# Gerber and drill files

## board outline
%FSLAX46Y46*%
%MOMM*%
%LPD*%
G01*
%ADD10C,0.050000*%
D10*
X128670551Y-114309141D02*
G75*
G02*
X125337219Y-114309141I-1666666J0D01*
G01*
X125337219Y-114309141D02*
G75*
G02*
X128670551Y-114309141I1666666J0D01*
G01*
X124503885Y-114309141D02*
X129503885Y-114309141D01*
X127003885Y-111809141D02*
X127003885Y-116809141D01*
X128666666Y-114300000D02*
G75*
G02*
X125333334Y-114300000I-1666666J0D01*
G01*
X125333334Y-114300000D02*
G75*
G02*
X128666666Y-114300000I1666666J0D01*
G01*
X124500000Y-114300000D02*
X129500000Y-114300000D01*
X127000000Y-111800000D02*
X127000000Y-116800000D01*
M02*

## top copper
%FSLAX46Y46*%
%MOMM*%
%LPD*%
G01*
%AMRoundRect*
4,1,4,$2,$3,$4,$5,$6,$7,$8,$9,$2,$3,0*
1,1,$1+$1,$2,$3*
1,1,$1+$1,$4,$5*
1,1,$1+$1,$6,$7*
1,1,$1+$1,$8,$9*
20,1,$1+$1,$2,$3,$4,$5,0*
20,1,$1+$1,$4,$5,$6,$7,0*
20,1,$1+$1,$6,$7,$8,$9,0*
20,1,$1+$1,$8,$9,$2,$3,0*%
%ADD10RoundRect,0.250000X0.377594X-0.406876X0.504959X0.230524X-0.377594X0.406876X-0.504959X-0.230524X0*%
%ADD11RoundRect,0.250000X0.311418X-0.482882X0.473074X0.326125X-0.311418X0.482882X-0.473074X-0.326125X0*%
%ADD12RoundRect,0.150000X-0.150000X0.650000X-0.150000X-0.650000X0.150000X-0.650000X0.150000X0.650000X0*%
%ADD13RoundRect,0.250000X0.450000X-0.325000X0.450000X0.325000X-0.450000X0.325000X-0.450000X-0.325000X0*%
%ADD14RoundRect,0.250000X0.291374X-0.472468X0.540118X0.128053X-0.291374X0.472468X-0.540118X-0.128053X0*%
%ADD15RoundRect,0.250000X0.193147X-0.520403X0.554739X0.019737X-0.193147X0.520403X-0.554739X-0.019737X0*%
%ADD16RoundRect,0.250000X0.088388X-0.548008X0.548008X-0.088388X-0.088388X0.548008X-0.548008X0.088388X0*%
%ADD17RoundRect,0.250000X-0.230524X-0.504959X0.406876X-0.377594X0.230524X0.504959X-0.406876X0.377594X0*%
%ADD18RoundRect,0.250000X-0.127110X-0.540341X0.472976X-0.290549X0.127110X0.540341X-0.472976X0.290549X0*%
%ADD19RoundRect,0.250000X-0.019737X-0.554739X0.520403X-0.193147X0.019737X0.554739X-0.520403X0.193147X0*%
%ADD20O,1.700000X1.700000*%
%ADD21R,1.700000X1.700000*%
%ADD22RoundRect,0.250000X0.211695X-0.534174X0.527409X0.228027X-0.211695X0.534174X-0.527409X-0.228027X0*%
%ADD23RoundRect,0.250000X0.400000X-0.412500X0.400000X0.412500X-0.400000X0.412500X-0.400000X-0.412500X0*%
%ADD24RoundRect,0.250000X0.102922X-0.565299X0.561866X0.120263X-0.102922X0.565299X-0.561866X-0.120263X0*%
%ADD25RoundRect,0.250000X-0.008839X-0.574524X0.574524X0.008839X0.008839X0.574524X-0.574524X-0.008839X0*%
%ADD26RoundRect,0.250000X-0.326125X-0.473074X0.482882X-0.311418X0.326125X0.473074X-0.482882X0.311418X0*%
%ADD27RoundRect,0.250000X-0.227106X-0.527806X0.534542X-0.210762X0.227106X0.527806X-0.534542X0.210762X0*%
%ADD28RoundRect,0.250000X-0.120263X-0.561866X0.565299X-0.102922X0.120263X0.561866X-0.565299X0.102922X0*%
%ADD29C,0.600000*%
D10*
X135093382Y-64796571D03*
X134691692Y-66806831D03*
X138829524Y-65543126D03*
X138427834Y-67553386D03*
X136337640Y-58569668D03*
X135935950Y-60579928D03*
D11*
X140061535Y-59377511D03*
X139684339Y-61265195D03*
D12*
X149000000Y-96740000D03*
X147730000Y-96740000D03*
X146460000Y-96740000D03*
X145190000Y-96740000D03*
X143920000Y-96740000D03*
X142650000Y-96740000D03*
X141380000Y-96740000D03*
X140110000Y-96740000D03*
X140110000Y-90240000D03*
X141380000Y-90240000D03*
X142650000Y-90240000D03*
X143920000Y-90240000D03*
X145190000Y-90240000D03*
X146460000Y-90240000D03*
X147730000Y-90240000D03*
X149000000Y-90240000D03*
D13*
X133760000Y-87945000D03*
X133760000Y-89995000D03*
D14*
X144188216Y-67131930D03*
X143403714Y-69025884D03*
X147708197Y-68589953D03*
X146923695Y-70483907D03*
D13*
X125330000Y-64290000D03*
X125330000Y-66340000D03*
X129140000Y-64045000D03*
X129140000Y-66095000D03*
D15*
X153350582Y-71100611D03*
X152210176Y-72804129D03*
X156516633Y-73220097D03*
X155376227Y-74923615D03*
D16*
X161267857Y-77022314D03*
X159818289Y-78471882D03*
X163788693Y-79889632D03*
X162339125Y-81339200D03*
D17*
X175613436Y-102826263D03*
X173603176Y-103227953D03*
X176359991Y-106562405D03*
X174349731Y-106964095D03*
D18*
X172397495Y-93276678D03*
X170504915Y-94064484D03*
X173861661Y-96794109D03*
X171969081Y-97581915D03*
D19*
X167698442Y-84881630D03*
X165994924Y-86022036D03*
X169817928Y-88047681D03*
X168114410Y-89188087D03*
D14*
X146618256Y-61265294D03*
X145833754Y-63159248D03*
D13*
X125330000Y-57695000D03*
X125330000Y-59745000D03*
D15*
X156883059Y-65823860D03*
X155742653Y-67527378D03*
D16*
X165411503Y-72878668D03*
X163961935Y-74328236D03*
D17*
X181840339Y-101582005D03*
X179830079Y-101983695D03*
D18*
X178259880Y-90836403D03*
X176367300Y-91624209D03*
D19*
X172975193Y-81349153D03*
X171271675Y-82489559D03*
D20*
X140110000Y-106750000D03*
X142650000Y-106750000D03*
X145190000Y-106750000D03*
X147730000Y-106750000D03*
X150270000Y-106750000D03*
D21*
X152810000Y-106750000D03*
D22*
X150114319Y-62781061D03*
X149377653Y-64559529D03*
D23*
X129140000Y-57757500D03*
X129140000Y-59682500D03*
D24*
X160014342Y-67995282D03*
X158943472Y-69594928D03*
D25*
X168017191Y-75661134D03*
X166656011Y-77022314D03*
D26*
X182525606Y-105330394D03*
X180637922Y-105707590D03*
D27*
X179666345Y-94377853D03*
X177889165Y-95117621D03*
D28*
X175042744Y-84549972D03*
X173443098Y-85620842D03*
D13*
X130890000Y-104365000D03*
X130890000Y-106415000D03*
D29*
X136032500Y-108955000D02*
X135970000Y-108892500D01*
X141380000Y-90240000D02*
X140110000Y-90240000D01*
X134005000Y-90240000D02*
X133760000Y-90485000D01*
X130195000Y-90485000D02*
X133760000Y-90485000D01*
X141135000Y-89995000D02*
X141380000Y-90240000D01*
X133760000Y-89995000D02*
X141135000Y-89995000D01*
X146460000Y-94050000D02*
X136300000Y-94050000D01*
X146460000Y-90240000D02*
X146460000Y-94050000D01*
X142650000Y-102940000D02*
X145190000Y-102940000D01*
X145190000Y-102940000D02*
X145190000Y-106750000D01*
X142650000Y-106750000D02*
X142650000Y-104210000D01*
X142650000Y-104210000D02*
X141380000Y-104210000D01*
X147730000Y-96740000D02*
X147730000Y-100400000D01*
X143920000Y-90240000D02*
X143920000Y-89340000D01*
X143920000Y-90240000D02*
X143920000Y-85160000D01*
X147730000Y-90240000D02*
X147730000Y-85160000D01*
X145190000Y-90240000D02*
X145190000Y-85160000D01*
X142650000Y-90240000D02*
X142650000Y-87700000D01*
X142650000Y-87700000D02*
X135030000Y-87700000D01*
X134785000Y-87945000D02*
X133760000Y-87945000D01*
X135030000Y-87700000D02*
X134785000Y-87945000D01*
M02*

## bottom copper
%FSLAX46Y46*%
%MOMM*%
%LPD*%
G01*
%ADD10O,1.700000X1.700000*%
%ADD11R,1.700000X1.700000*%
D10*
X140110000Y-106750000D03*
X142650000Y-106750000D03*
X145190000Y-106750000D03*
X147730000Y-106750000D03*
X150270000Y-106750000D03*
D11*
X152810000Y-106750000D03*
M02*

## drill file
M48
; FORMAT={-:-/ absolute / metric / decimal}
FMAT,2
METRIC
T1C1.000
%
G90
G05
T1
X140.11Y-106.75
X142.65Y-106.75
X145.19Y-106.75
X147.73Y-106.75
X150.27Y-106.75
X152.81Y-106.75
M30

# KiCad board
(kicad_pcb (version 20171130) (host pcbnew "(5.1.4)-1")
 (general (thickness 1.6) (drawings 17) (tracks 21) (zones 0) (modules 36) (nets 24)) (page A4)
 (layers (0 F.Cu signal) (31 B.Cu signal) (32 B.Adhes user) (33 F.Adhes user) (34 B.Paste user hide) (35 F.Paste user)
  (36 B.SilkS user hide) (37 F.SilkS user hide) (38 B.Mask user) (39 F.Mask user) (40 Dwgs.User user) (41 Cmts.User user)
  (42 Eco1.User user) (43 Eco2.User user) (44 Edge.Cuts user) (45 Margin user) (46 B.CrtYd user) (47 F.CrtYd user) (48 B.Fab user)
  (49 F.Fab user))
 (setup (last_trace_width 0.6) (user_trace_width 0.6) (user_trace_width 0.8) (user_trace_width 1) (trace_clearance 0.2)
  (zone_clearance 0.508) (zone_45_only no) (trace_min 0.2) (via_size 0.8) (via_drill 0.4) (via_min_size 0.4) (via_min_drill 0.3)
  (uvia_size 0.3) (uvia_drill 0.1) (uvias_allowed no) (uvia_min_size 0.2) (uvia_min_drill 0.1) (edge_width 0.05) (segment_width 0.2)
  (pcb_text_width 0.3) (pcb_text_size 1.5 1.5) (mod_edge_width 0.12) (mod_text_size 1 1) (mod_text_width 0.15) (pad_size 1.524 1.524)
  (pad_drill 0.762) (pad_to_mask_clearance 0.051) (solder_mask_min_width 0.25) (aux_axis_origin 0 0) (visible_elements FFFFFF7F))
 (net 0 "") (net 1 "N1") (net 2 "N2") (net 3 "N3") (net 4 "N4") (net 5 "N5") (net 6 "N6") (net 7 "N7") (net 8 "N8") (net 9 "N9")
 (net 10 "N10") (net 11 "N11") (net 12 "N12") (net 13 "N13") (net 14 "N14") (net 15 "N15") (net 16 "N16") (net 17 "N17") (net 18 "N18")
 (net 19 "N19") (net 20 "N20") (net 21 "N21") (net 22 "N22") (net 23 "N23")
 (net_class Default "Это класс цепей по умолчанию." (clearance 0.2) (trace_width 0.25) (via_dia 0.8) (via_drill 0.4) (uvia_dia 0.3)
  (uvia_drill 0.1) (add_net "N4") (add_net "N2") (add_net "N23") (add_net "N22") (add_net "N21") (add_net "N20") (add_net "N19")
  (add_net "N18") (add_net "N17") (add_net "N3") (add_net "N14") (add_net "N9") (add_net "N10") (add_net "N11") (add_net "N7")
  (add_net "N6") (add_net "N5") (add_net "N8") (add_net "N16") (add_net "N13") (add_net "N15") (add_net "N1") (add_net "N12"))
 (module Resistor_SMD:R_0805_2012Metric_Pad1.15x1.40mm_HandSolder (layer F.Cu) (at 134.892537 65.801701 78.7)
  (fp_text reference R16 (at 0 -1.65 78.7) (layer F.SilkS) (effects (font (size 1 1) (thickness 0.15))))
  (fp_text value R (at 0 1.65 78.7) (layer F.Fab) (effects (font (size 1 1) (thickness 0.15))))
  (pad 2 smd roundrect (at 1.025 0 78.7) (size 1.15 1.4) (layers F.Cu F.Paste F.Mask) (roundrect_rratio 0.217391) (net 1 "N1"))
  (pad 1 smd roundrect (at -1.025 0 78.7) (size 1.15 1.4) (layers F.Cu F.Paste F.Mask) (roundrect_rratio 0.217391) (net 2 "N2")))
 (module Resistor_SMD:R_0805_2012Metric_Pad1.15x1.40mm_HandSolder (layer F.Cu) (at 138.628679 66.548256 78.7)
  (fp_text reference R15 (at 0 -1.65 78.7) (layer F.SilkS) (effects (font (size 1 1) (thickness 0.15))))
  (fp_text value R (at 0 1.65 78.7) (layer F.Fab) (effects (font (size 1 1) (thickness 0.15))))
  (pad 2 smd roundrect (at 1.025 0 78.7) (size 1.15 1.4) (layers F.Cu F.Paste F.Mask) (roundrect_rratio 0.217391) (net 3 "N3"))
  (pad 1 smd roundrect (at -1.025 0 78.7) (size 1.15 1.4) (layers F.Cu F.Paste F.Mask) (roundrect_rratio 0.217391) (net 2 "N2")))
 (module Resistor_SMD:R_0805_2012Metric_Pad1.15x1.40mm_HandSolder (layer F.Cu) (at 136.136795 59.574798 78.7)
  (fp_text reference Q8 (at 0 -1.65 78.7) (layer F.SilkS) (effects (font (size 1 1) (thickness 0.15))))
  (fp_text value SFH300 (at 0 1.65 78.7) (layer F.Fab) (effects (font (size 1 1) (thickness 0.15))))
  (pad 2 smd roundrect (at 1.025 0 78.7) (size 1.15 1.4) (layers F.Cu F.Paste F.Mask) (roundrect_rratio 0.217391) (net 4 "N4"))
  (pad 1 smd roundrect (at -1.025 0 78.7) (size 1.15 1.4) (layers F.Cu F.Paste F.Mask) (roundrect_rratio 0.217391) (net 1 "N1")))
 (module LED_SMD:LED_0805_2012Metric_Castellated (layer F.Cu) (at 139.872937 60.321353 78.7)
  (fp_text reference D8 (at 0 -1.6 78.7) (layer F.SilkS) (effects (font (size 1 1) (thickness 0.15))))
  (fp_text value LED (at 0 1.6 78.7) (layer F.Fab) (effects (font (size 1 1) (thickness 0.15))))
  (pad 2 smd roundrect (at 0.9625 0 78.7) (size 1.325 1.3) (layers F.Cu F.Paste F.Mask) (roundrect_rratio 0.192308) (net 4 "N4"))
  (pad 1 smd roundrect (at -0.9625 0 78.7) (size 1.325 1.3) (layers F.Cu F.Paste F.Mask) (roundrect_rratio 0.192308) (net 3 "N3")))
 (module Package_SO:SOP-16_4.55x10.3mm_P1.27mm (layer F.Cu) (at 144.555 93.49 270)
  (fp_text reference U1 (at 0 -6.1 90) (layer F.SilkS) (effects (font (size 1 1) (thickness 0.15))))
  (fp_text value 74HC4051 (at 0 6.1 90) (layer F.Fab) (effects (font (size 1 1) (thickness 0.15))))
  (pad 16 smd roundrect (at 3.25 -4.445 270) (size 1.6 0.6) (layers F.Cu F.Paste F.Mask) (roundrect_rratio 0.25) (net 4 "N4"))
  (pad 15 smd roundrect (at 3.25 -3.175 270) (size 1.6 0.6) (layers F.Cu F.Paste F.Mask) (roundrect_rratio 0.25) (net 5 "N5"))
  (pad 14 smd roundrect (at 3.25 -1.905 270) (size 1.6 0.6) (layers F.Cu F.Paste F.Mask) (roundrect_rratio 0.25) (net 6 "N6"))
  (pad 13 smd roundrect (at 3.25 -0.635 270) (size 1.6 0.6) (layers F.Cu F.Paste F.Mask) (roundrect_rratio 0.25) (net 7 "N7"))
  (pad 12 smd roundrect (at 3.25 0.635 270) (size 1.6 0.6) (layers F.Cu F.Paste F.Mask) (roundrect_rratio 0.25) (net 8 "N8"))
  (pad 11 smd roundrect (at 3.25 1.905 270) (size 1.6 0.6) (layers F.Cu F.Paste F.Mask) (roundrect_rratio 0.25) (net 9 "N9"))
  (pad 10 smd roundrect (at 3.25 3.175 270) (size 1.6 0.6) (layers F.Cu F.Paste F.Mask) (roundrect_rratio 0.25) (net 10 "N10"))
  (pad 9 smd roundrect (at 3.25 4.445 270) (size 1.6 0.6) (layers F.Cu F.Paste F.Mask) (roundrect_rratio 0.25) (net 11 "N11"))
  (pad 8 smd roundrect (at -3.25 4.445 270) (size 1.6 0.6) (layers F.Cu F.Paste F.Mask) (roundrect_rratio 0.25) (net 2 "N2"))
  (pad 7 smd roundrect (at -3.25 3.175 270) (size 1.6 0.6) (layers F.Cu F.Paste F.Mask) (roundrect_rratio 0.25) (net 2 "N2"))
  (pad 6 smd roundrect (at -3.25 1.905 270) (size 1.6 0.6) (layers F.Cu F.Paste F.Mask) (roundrect_rratio 0.25) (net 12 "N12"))
  (pad 5 smd roundrect (at -3.25 0.635 270) (size 1.6 0.6) (layers F.Cu F.Paste F.Mask) (roundrect_rratio 0.25) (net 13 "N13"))
  (pad 4 smd roundrect (at -3.25 -0.635 270) (size 1.6 0.6) (layers F.Cu F.Paste F.Mask) (roundrect_rratio 0.25) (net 1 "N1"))
  (pad 3 smd roundrect (at -3.25 -1.905 270) (size 1.6 0.6) (layers F.Cu F.Paste F.Mask) (roundrect_rratio 0.25) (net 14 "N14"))
  (pad 2 smd roundrect (at -3.25 -3.175 270) (size 1.6 0.6) (layers F.Cu F.Paste F.Mask) (roundrect_rratio 0.25) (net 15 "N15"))
  (pad 1 smd roundrect (at -3.25 -4.445 270) (size 1.6 0.6) (layers F.Cu F.Paste F.Mask) (roundrect_rratio 0.25) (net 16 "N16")))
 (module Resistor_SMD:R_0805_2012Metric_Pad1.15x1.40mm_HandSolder (layer F.Cu) (at 133.76 88.97 90)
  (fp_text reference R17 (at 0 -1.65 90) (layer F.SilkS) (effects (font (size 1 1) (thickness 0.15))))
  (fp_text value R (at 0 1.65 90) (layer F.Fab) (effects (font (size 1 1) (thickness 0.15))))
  (pad 2 smd roundrect (at 1.025 0 90) (size 1.15 1.4) (layers F.Cu F.Paste F.Mask) (roundrect_rratio 0.217391) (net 12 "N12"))
  (pad 1 smd roundrect (at -1.025 0 90) (size 1.15 1.4) (layers F.Cu F.Paste F.Mask) (roundrect_rratio 0.217391) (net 2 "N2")))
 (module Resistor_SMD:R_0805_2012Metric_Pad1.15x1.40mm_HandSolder (layer F.Cu) (at 143.795965 68.078907 67.5)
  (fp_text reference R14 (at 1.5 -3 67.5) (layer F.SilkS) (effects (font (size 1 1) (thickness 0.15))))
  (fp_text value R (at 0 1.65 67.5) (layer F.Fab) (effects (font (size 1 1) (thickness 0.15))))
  (pad 2 smd roundrect (at 1.025 0 67.5) (size 1.15 1.4) (layers F.Cu F.Paste F.Mask) (roundrect_rratio 0.217391) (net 15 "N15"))
  (pad 1 smd roundrect (at -1.025 0 67.5) (size 1.15 1.4) (layers F.Cu F.Paste F.Mask) (roundrect_rratio 0.217391) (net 2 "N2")))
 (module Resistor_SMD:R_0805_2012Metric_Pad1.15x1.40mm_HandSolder (layer F.Cu) (at 147.315946 69.53693 67.5)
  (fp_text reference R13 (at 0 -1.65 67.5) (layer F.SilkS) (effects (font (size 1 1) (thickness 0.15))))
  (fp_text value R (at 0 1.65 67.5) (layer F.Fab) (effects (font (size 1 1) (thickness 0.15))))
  (pad 2 smd roundrect (at 1.025 0 67.5) (size 1.15 1.4) (layers F.Cu F.Paste F.Mask) (roundrect_rratio 0.217391) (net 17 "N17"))
  (pad 1 smd roundrect (at -1.025 0 67.5) (size 1.15 1.4) (layers F.Cu F.Paste F.Mask) (roundrect_rratio 0.217391) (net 2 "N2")))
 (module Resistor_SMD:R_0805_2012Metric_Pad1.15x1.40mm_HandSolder (layer F.Cu) (at 125.33 65.315 90)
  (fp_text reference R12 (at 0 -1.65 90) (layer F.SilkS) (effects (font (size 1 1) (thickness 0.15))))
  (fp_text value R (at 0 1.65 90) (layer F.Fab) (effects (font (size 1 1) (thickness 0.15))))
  (pad 2 smd roundrect (at 1.025 0 90) (size 1.15 1.4) (layers F.Cu F.Paste F.Mask) (roundrect_rratio 0.217391) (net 13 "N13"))
  (pad 1 smd roundrect (at -1.025 0 90) (size 1.15 1.4) (layers F.Cu F.Paste F.Mask) (roundrect_rratio 0.217391) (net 2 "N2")))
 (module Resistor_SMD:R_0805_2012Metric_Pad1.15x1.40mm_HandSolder (layer F.Cu) (at 129.14 65.07 90)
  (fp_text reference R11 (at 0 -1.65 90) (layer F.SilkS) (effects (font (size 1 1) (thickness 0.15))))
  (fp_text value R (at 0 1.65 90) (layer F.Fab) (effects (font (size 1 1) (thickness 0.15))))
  (pad 2 smd roundrect (at 1.025 0 90) (size 1.15 1.4) (layers F.Cu F.Paste F.Mask) (roundrect_rratio 0.217391) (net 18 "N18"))
  (pad 1 smd roundrect (at -1.025 0 90) (size 1.15 1.4) (layers F.Cu F.Paste F.Mask) (roundrect_rratio 0.217391) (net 2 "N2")))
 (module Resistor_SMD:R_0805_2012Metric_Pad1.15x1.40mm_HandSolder (layer F.Cu) (at 152.780379 71.95237 56.2)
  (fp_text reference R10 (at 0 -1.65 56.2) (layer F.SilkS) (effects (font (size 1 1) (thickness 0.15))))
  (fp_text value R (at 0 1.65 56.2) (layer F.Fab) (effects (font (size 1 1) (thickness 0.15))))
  (pad 2 smd roundrect (at 1.025 0 56.2) (size 1.15 1.4) (layers F.Cu F.Paste F.Mask) (roundrect_rratio 0.217391) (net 16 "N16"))
  (pad 1 smd roundrect (at -1.025 0 56.2) (size 1.15 1.4) (layers F.Cu F.Paste F.Mask) (roundrect_rratio 0.217391) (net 2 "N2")))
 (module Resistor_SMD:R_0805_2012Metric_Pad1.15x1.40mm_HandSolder (layer F.Cu) (at 155.94643 74.071856 56.2)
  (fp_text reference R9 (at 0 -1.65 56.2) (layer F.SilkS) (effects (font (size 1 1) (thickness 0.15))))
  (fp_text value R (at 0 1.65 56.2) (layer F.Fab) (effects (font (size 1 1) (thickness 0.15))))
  (pad 2 smd roundrect (at 1.025 0 56.2) (size 1.15 1.4) (layers F.Cu F.Paste F.Mask) (roundrect_rratio 0.217391) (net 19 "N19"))
  (pad 1 smd roundrect (at -1.025 0 56.2) (size 1.15 1.4) (layers F.Cu F.Paste F.Mask) (roundrect_rratio 0.217391) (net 2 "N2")))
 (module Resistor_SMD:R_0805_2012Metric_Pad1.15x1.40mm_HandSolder (layer F.Cu) (at 160.543073 77.747098 45)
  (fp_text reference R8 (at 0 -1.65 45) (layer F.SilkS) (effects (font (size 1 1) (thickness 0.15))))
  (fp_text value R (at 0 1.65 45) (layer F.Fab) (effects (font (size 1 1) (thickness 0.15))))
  (pad 2 smd roundrect (at 1.025 0 45) (size 1.15 1.4) (layers F.Cu F.Paste F.Mask) (roundrect_rratio 0.217391) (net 8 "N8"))
  (pad 1 smd roundrect (at -1.025 0 45) (size 1.15 1.4) (layers F.Cu F.Paste F.Mask) (roundrect_rratio 0.217391) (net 2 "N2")))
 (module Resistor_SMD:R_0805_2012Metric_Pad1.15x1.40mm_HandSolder (layer F.Cu) (at 163.063909 80.614416 45)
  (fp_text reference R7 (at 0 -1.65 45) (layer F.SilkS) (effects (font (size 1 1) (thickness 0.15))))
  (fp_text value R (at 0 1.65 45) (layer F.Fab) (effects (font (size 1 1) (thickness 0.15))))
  (pad 2 smd roundrect (at 1.025 0 45) (size 1.15 1.4) (layers F.Cu F.Paste F.Mask) (roundrect_rratio 0.217391) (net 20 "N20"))
  (pad 1 smd roundrect (at -1.025 0 45) (size 1.15 1.4) (layers F.Cu F.Paste F.Mask) (roundrect_rratio 0.217391) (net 2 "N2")))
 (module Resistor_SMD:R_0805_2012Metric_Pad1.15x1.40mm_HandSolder (layer F.Cu) (at 174.608306 103.027108 11.3)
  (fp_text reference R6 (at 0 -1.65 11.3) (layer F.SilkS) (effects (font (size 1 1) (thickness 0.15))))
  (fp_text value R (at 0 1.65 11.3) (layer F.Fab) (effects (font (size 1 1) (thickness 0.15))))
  (pad 2 smd roundrect (at 1.025 0 11.3) (size 1.15 1.4) (layers F.Cu F.Paste F.Mask) (roundrect_rratio 0.217391) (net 5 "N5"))
  (pad 1 smd roundrect (at -1.025 0 11.3) (size 1.15 1.4) (layers F.Cu F.Paste F.Mask) (roundrect_rratio 0.217391) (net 2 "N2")))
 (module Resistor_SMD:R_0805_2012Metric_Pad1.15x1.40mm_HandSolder (layer F.Cu) (at 175.354861 106.76325 11.3)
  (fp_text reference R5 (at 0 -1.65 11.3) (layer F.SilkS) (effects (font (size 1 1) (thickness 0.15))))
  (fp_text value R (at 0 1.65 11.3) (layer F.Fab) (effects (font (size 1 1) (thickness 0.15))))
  (pad 2 smd roundrect (at 1.025 0 11.3) (size 1.15 1.4) (layers F.Cu F.Paste F.Mask) (roundrect_rratio 0.217391) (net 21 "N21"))
  (pad 1 smd roundrect (at -1.025 0 11.3) (size 1.15 1.4) (layers F.Cu F.Paste F.Mask) (roundrect_rratio 0.217391) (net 2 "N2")))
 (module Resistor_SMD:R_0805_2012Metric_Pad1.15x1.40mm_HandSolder (layer F.Cu) (at 171.451205 93.670581 22.6)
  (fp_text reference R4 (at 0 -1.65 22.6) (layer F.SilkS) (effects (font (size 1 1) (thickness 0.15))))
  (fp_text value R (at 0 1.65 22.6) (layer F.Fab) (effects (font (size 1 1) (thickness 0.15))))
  (pad 2 smd roundrect (at 1.025 0 22.6) (size 1.15 1.4) (layers F.Cu F.Paste F.Mask) (roundrect_rratio 0.217391) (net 6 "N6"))
  (pad 1 smd roundrect (at -1.025 0 22.6) (size 1.15 1.4) (layers F.Cu F.Paste F.Mask) (roundrect_rratio 0.217391) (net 2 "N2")))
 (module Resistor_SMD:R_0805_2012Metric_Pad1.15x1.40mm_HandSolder (layer F.Cu) (at 172.915371 97.188012 22.6)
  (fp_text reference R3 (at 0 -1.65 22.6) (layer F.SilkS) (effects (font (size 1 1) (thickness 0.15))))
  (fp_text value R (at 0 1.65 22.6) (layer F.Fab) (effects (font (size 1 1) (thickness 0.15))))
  (pad 2 smd roundrect (at 1.025 0 22.6) (size 1.15 1.4) (layers F.Cu F.Paste F.Mask) (roundrect_rratio 0.217391) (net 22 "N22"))
  (pad 1 smd roundrect (at -1.025 0 22.6) (size 1.15 1.4) (layers F.Cu F.Paste F.Mask) (roundrect_rratio 0.217391) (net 2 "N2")))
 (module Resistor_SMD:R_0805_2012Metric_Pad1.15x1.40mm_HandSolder (layer F.Cu) (at 166.846683 85.451833 33.8)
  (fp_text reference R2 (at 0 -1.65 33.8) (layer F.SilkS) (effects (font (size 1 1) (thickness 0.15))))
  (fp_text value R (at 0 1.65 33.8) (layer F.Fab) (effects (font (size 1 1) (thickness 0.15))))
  (pad 2 smd roundrect (at 1.025 0 33.8) (size 1.15 1.4) (layers F.Cu F.Paste F.Mask) (roundrect_rratio 0.217391) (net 7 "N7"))
  (pad 1 smd roundrect (at -1.025 0 33.8) (size 1.15 1.4) (layers F.Cu F.Paste F.Mask) (roundrect_rratio 0.217391) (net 2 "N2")))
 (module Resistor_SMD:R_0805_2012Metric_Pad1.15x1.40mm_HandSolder (layer F.Cu) (at 168.966169 88.617884 33.8)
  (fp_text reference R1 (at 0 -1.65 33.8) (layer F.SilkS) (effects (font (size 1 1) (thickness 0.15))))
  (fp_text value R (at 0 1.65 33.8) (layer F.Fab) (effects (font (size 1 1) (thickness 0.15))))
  (pad 2 smd roundrect (at 1.025 0 33.8) (size 1.15 1.4) (layers F.Cu F.Paste F.Mask) (roundrect_rratio 0.217391) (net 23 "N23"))
  (pad 1 smd roundrect (at -1.025 0 33.8) (size 1.15 1.4) (layers F.Cu F.Paste F.Mask) (roundrect_rratio 0.217391) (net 2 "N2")))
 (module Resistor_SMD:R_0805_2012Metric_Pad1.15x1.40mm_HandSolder (layer F.Cu) (at 146.226005 62.212271 67.5)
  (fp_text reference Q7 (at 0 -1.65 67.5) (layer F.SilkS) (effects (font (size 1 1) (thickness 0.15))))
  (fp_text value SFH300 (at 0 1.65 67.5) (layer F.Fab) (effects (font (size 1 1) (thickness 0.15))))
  (pad 2 smd roundrect (at 1.025 0 67.5) (size 1.15 1.4) (layers F.Cu F.Paste F.Mask) (roundrect_rratio 0.217391) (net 4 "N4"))
  (pad 1 smd roundrect (at -1.025 0 67.5) (size 1.15 1.4) (layers F.Cu F.Paste F.Mask) (roundrect_rratio 0.217391) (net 15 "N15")))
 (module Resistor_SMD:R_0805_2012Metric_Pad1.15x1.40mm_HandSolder (layer F.Cu) (at 125.33 58.72 90)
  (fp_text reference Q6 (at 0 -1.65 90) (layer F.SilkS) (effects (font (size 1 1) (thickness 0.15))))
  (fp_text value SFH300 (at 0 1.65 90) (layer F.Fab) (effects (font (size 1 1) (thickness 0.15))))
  (pad 2 smd roundrect (at 1.025 0 90) (size 1.15 1.4) (layers F.Cu F.Paste F.Mask) (roundrect_rratio 0.217391) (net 4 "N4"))
  (pad 1 smd roundrect (at -1.025 0 90) (size 1.15 1.4) (layers F.Cu F.Paste F.Mask) (roundrect_rratio 0.217391) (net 13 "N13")))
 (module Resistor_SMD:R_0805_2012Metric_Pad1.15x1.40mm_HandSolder (layer F.Cu) (at 156.312856 66.675619 56.2)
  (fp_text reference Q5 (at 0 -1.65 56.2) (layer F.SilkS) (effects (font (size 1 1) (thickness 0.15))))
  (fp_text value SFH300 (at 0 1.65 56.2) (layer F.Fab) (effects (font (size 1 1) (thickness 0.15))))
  (pad 2 smd roundrect (at 1.025 0 56.2) (size 1.15 1.4) (layers F.Cu F.Paste F.Mask) (roundrect_rratio 0.217391) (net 4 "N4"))
  (pad 1 smd roundrect (at -1.025 0 56.2) (size 1.15 1.4) (layers F.Cu F.Paste F.Mask) (roundrect_rratio 0.217391) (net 16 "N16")))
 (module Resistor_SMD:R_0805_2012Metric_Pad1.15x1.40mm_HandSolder (layer F.Cu) (at 164.686719 73.603452 45)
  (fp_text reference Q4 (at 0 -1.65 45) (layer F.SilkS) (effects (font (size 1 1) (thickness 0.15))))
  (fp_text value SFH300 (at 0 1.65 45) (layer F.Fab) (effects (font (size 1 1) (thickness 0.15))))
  (pad 2 smd roundrect (at 1.025 0 45) (size 1.15 1.4) (layers F.Cu F.Paste F.Mask) (roundrect_rratio 0.217391) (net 4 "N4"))
  (pad 1 smd roundrect (at -1.025 0 45) (size 1.15 1.4) (layers F.Cu F.Paste F.Mask) (roundrect_rratio 0.217391) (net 8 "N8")))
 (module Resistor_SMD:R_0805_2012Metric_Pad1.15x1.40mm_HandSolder (layer F.Cu) (at 180.835209 101.78285 11.3)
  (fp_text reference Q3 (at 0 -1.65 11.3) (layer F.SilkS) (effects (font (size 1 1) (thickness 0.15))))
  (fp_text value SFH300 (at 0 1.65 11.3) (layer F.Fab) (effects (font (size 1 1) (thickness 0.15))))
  (pad 2 smd roundrect (at 1.025 0 11.3) (size 1.15 1.4) (layers F.Cu F.Paste F.Mask) (roundrect_rratio 0.217391) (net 4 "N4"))
  (pad 1 smd roundrect (at -1.025 0 11.3) (size 1.15 1.4) (layers F.Cu F.Paste F.Mask) (roundrect_rratio 0.217391) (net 5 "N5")))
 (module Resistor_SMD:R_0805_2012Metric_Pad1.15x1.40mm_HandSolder (layer F.Cu) (at 177.31359 91.230306 22.6)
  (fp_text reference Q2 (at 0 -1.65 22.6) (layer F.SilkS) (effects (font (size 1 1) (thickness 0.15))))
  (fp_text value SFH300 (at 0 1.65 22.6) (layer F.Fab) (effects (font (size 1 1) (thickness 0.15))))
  (pad 2 smd roundrect (at 1.025 0 22.6) (size 1.15 1.4) (layers F.Cu F.Paste F.Mask) (roundrect_rratio 0.217391) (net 4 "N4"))
  (pad 1 smd roundrect (at -1.025 0 22.6) (size 1.15 1.4) (layers F.Cu F.Paste F.Mask) (roundrect_rratio 0.217391) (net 6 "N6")))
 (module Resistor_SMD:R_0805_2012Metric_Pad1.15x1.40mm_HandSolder (layer F.Cu) (at 172.123434 81.919356 33.8)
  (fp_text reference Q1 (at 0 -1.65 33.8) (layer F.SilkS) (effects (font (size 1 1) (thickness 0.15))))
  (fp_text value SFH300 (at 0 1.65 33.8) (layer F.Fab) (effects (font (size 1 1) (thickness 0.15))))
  (pad 2 smd roundrect (at 1.025 0 33.8) (size 1.15 1.4) (layers F.Cu F.Paste F.Mask) (roundrect_rratio 0.217391) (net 4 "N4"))
  (pad 1 smd roundrect (at -1.025 0 33.8) (size 1.15 1.4) (layers F.Cu F.Paste F.Mask) (roundrect_rratio 0.217391) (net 7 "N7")))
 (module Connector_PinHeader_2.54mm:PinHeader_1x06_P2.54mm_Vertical (layer F.Cu) (at 152.81 106.75 270)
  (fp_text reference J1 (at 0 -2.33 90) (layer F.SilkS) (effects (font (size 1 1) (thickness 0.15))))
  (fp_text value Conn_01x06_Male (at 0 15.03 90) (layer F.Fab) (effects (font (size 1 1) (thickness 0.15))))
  (pad 6 thru_hole oval (at 0 12.7 270) (size 1.7 1.7) (drill 1) (layers *.Cu *.Mask) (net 11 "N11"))
  (pad 5 thru_hole oval (at 0 10.16 270) (size 1.7 1.7) (drill 1) (layers *.Cu *.Mask) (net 10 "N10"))
  (pad 4 thru_hole oval (at 0 7.62 270) (size 1.7 1.7) (drill 1) (layers *.Cu *.Mask) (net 9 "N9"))
  (pad 3 thru_hole oval (at 0 5.08 270) (size 1.7 1.7) (drill 1) (layers *.Cu *.Mask) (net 14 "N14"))
  (pad 2 thru_hole oval (at 0 2.54 270) (size 1.7 1.7) (drill 1) (layers *.Cu *.Mask) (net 4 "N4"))
  (pad 1 thru_hole rect (at 0 0 270) (size 1.7 1.7) (drill 1) (layers *.Cu *.Mask) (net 2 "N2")))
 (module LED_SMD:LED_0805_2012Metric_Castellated (layer F.Cu) (at 149.745986 63.670295 67.5)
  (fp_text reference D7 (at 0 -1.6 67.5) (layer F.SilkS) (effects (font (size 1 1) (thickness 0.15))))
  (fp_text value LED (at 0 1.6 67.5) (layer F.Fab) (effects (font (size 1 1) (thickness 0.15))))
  (pad 2 smd roundrect (at 0.9625 0 67.5) (size 1.325 1.3) (layers F.Cu F.Paste F.Mask) (roundrect_rratio 0.192308) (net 4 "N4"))
  (pad 1 smd roundrect (at -0.9625 0 67.5) (size 1.325 1.3) (layers F.Cu F.Paste F.Mask) (roundrect_rratio 0.192308) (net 17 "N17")))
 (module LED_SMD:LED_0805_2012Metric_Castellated (layer F.Cu) (at 129.14 58.72 90)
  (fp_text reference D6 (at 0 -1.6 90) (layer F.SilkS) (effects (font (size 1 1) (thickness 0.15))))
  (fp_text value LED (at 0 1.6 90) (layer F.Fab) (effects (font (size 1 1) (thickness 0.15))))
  (pad 2 smd roundrect (at 0.9625 0 90) (size 1.325 1.3) (layers F.Cu F.Paste F.Mask) (roundrect_rratio 0.192308) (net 4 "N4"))
  (pad 1 smd roundrect (at -0.9625 0 90) (size 1.325 1.3) (layers F.Cu F.Paste F.Mask) (roundrect_rratio 0.192308) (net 18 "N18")))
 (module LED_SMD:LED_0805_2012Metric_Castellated (layer F.Cu) (at 159.478907 68.795105 56.2)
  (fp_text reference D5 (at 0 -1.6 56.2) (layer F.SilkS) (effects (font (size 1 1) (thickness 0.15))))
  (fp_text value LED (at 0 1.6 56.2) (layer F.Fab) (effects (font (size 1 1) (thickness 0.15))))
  (pad 2 smd roundrect (at 0.9625 0 56.2) (size 1.325 1.3) (layers F.Cu F.Paste F.Mask) (roundrect_rratio 0.192308) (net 4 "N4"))
  (pad 1 smd roundrect (at -0.9625 0 56.2) (size 1.325 1.3) (layers F.Cu F.Paste F.Mask) (roundrect_rratio 0.192308) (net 19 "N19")))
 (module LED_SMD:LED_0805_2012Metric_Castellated (layer F.Cu) (at 167.336601 76.341724 45)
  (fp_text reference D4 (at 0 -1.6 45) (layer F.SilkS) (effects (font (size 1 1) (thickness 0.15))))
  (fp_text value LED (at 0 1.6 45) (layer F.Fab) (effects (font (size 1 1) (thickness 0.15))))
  (pad 2 smd roundrect (at 0.9625 0 45) (size 1.325 1.3) (layers F.Cu F.Paste F.Mask) (roundrect_rratio 0.192308) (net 4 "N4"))
  (pad 1 smd roundrect (at -0.9625 0 45) (size 1.325 1.3) (layers F.Cu F.Paste F.Mask) (roundrect_rratio 0.192308) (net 20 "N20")))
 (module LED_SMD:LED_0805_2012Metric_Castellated (layer F.Cu) (at 181.581764 105.518992 11.3)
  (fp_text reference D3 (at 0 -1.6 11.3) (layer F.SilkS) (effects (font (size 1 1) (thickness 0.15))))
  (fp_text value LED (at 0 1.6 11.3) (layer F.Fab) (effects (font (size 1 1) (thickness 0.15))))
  (pad 2 smd roundrect (at 0.9625 0 11.3) (size 1.325 1.3) (layers F.Cu F.Paste F.Mask) (roundrect_rratio 0.192308) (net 4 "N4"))
  (pad 1 smd roundrect (at -0.9625 0 11.3) (size 1.325 1.3) (layers F.Cu F.Paste F.Mask) (roundrect_rratio 0.192308) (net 21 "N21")))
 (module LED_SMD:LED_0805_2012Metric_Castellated (layer F.Cu) (at 178.777755 94.747737 22.6)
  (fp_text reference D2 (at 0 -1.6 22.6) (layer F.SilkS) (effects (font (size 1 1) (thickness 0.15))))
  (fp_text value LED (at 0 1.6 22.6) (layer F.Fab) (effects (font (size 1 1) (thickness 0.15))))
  (pad 2 smd roundrect (at 0.9625 0 22.6) (size 1.325 1.3) (layers F.Cu F.Paste F.Mask) (roundrect_rratio 0.192308) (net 4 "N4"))
  (pad 1 smd roundrect (at -0.9625 0 22.6) (size 1.325 1.3) (layers F.Cu F.Paste F.Mask) (roundrect_rratio 0.192308) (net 22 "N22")))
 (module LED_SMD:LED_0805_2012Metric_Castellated (layer F.Cu) (at 174.242921 85.085407 33.8)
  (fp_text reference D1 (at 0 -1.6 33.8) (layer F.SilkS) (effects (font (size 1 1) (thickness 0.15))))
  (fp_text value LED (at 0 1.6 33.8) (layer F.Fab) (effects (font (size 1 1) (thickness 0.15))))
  (pad 2 smd roundrect (at 0.9625 0 33.8) (size 1.325 1.3) (layers F.Cu F.Paste F.Mask) (roundrect_rratio 0.192308) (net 4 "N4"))
  (pad 1 smd roundrect (at -0.9625 0 33.8) (size 1.325 1.3) (layers F.Cu F.Paste F.Mask) (roundrect_rratio 0.192308) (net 23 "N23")))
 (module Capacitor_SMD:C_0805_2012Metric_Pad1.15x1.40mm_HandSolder (layer F.Cu) (at 130.89 105.39 90)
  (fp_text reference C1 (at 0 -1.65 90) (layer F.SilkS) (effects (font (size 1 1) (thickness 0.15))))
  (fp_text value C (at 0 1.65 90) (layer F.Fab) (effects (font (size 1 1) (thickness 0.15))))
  (pad 2 smd roundrect (at 1.025 0 90) (size 1.15 1.4) (layers F.Cu F.Paste F.Mask) (roundrect_rratio 0.217391) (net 2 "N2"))
  (pad 1 smd roundrect (at -1.025 0 90) (size 1.15 1.4) (layers F.Cu F.Paste F.Mask) (roundrect_rratio 0.217391) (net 4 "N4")))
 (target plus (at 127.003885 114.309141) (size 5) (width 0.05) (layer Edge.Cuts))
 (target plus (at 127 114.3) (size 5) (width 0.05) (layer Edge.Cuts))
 (segment (start 136.0325 108.955) (end 135.97 108.8925) (width 0.6) (layer F.Cu) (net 4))
 (segment (start 141.38 90.24) (end 140.11 90.24) (width 0.6) (layer F.Cu) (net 2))
 (segment (start 134.005 90.24) (end 133.76 90.485) (width 0.6) (layer F.Cu) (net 2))
 (segment (start 130.195 90.485) (end 133.76 90.485) (width 0.6) (layer F.Cu) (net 2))
 (segment (start 141.135 89.995) (end 141.38 90.24) (width 0.6) (layer F.Cu) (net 2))
 (segment (start 133.76 89.995) (end 141.135 89.995) (width 0.6) (layer F.Cu) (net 2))
 (segment (start 146.46 94.05) (end 136.3 94.05) (width 0.6) (layer F.Cu) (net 14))
 (segment (start 146.46 90.24) (end 146.46 94.05) (width 0.6) (layer F.Cu) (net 14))
 (segment (start 142.65 102.94) (end 145.19 102.94) (width 0.6) (layer F.Cu) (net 9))
 (segment (start 145.19 102.94) (end 145.19 106.75) (width 0.6) (layer F.Cu) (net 9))
 (segment (start 142.65 106.75) (end 142.65 104.21) (width 0.6) (layer F.Cu) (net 10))
 (segment (start 142.65 104.21) (end 141.38 104.21) (width 0.6) (layer F.Cu) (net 10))
 (segment (start 147.73 96.74) (end 147.73 100.4) (width 0.6) (layer F.Cu) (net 5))
 (segment (start 143.92 90.24) (end 143.92 89.34) (width 0.6) (layer F.Cu) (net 13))
 (segment (start 143.92 90.24) (end 143.92 85.16) (width 0.6) (layer F.Cu) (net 13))
 (segment (start 147.73 90.24) (end 147.73 85.16) (width 0.6) (layer F.Cu) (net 15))
 (segment (start 145.19 90.24) (end 145.19 85.16) (width 0.6) (layer F.Cu) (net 1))
 (segment (start 142.65 90.24) (end 142.65 87.7) (width 0.6) (layer F.Cu) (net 12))
 (segment (start 142.65 87.7) (end 135.03 87.7) (width 0.6) (layer F.Cu) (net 12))
 (segment (start 134.785 87.945) (end 133.76 87.945) (width 0.6) (layer F.Cu) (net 12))
 (segment (start 135.03 87.7) (end 134.785 87.945) (width 0.6) (layer F.Cu) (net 12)))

